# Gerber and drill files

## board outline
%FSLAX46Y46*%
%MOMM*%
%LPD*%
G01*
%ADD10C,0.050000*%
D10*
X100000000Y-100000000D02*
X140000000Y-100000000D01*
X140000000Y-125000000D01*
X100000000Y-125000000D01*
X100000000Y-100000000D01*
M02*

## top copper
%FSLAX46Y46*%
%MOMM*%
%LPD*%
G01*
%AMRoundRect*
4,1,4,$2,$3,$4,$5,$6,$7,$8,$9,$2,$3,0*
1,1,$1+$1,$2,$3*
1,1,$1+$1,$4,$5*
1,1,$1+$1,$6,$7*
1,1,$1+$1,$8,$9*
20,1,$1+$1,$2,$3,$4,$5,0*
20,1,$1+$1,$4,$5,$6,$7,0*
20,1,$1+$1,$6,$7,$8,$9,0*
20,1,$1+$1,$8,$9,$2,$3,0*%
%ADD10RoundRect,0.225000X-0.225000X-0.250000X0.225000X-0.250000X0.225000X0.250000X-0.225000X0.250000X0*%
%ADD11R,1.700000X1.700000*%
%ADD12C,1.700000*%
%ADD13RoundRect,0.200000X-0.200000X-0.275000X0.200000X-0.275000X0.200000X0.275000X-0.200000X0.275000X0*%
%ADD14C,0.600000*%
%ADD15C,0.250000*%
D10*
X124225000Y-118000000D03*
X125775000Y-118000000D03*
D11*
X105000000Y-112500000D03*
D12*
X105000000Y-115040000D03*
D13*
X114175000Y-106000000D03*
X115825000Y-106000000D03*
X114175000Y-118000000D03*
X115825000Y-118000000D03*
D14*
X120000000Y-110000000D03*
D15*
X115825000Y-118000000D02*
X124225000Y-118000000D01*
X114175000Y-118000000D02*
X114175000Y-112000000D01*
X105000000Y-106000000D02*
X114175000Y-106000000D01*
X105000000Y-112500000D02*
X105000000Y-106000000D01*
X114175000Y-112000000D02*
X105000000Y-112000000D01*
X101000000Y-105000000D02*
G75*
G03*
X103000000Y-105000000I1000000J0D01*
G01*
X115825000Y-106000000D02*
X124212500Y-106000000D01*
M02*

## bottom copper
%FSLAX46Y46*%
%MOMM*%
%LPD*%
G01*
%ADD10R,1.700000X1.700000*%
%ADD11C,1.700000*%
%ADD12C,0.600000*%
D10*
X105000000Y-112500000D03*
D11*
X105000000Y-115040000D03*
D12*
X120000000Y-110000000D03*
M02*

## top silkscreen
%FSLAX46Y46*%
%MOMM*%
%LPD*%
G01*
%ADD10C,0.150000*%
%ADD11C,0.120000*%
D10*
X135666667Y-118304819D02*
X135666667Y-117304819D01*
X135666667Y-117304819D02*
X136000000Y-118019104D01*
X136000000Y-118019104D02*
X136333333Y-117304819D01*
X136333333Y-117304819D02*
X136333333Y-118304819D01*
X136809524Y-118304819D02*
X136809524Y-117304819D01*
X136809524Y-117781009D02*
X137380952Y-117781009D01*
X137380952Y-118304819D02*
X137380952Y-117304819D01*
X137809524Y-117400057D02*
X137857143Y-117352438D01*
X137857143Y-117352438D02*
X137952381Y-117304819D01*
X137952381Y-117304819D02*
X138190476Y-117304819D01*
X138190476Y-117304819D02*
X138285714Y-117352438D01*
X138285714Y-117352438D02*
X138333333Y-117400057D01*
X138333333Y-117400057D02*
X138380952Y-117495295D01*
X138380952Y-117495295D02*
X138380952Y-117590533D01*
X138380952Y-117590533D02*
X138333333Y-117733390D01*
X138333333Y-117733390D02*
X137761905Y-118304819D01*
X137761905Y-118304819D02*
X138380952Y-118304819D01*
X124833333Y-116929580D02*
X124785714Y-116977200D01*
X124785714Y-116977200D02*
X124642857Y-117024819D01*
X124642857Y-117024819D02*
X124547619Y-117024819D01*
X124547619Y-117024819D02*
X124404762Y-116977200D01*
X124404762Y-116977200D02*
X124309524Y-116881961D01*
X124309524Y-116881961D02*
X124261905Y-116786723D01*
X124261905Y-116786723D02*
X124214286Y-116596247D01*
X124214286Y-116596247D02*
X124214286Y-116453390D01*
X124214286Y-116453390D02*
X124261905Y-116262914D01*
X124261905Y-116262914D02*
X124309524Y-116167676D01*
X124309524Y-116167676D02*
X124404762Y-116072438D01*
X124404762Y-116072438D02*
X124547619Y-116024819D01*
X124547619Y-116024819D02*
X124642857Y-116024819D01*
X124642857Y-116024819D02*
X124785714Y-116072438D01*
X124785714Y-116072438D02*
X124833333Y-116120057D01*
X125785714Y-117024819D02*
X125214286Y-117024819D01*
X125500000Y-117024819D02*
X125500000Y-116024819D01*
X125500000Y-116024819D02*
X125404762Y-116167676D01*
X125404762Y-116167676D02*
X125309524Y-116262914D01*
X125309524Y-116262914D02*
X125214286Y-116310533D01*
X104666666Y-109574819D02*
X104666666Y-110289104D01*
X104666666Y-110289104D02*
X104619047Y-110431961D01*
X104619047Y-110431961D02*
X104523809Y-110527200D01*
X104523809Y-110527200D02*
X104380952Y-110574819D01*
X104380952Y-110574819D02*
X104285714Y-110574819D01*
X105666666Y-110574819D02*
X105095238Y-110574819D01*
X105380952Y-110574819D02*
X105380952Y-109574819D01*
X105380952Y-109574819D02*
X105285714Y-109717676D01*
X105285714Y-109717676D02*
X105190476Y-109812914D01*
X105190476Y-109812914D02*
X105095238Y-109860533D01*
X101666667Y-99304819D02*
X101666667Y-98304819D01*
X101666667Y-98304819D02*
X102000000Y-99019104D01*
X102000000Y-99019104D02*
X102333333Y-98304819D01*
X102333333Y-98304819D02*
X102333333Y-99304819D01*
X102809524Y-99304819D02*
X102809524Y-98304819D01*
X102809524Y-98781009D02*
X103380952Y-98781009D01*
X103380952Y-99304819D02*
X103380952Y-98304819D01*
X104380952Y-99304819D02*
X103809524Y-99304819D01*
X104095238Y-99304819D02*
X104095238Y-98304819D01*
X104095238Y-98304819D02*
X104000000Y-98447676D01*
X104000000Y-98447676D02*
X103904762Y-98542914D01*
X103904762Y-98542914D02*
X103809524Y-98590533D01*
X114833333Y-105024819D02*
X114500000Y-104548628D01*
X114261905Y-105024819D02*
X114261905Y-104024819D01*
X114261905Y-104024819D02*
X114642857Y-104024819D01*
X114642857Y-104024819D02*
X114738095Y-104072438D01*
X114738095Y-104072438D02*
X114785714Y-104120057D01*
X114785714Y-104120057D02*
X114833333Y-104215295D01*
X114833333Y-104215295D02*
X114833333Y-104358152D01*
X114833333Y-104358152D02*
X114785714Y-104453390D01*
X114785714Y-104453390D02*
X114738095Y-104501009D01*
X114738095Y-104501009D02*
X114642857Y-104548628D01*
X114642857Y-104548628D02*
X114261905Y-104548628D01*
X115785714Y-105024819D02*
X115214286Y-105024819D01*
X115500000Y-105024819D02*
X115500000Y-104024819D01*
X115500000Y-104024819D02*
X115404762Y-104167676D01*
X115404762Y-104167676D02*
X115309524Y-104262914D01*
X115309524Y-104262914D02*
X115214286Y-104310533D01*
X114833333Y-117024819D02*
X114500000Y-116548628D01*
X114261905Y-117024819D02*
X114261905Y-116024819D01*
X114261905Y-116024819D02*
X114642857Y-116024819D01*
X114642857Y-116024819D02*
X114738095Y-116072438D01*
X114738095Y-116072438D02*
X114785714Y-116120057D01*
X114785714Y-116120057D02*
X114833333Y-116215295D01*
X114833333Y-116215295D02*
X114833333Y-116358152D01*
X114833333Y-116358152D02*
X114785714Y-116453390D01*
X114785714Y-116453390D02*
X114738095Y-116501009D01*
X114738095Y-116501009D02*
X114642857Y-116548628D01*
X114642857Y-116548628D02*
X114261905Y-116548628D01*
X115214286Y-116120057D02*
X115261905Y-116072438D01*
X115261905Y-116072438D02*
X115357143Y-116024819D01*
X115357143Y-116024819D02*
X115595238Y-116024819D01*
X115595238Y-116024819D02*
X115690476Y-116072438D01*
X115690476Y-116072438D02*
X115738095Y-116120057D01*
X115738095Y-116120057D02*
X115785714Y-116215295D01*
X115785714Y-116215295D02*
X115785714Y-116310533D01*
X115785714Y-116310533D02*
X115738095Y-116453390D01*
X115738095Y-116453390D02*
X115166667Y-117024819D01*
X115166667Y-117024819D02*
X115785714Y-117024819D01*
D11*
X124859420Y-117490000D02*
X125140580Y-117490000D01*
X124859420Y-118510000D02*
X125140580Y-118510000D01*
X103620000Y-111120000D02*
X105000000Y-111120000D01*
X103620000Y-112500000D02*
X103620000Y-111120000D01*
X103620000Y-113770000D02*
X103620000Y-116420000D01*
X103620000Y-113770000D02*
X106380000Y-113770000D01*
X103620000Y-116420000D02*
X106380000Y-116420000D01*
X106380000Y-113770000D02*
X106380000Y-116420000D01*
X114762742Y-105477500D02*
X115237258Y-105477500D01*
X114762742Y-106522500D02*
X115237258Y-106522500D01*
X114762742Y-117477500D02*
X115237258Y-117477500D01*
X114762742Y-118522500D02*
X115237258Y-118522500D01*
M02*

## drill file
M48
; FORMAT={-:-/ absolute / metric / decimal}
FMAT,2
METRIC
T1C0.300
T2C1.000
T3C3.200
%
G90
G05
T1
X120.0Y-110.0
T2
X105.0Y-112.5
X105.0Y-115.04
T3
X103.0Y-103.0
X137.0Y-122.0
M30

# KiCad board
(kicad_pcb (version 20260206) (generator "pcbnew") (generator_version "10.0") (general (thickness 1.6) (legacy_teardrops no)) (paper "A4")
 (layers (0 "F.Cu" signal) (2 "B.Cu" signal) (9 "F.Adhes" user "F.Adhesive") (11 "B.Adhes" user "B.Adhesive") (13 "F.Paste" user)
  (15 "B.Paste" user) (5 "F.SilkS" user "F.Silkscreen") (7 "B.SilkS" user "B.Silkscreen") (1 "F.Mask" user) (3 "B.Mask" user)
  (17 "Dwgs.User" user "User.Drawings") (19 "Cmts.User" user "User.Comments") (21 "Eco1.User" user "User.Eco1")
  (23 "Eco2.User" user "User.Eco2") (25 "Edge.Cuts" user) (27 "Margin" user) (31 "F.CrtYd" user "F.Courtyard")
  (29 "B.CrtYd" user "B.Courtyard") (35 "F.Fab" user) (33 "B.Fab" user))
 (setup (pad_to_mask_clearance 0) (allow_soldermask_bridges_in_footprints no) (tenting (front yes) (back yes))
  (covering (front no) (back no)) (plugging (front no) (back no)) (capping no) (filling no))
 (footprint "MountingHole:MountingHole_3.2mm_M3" (layer "F.Cu") (at 137 122)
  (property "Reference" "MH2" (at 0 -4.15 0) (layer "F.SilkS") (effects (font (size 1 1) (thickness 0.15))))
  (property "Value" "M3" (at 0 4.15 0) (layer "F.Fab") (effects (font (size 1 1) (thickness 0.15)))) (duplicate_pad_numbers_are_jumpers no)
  (pad "" np_thru_hole circle (at 0 0) (size 3.2 3.2) (drill 3.2) (layers "*.Cu" "*.Mask")))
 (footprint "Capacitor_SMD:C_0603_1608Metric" (layer "F.Cu") (at 125 118)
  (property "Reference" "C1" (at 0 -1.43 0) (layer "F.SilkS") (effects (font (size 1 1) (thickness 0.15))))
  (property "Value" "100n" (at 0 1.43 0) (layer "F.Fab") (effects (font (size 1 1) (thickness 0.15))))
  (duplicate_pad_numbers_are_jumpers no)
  (fp_line (start -0.14058 -0.51) (end 0.14058 -0.51) (stroke (width 0.12) (type solid)) (layer "F.SilkS"))
  (fp_line (start -0.14058 0.51) (end 0.14058 0.51) (stroke (width 0.12) (type solid)) (layer "F.SilkS"))
  (pad "1" smd roundrect (at -0.775 0) (size 0.9 0.95) (layers "F.Cu" "F.Mask" "F.Paste") (roundrect_rratio 0.25) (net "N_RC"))
  (pad "2" smd roundrect (at 0.775 0) (size 0.9 0.95) (layers "F.Cu" "F.Mask" "F.Paste") (roundrect_rratio 0.25) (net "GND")))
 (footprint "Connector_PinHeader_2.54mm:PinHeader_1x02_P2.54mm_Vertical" (layer "F.Cu") (at 105 112.5)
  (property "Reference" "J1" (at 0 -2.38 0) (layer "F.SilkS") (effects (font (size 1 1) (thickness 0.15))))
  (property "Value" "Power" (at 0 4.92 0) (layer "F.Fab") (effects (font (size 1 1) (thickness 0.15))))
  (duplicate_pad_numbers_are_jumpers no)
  (fp_line (start -1.38 -1.38) (end 0 -1.38) (stroke (width 0.12) (type solid)) (layer "F.SilkS"))
  (fp_line (start -1.38 0) (end -1.38 -1.38) (stroke (width 0.12) (type solid)) (layer "F.SilkS"))
  (fp_line (start -1.38 1.27) (end -1.38 3.92) (stroke (width 0.12) (type solid)) (layer "F.SilkS"))
  (fp_line (start -1.38 1.27) (end 1.38 1.27) (stroke (width 0.12) (type solid)) (layer "F.SilkS"))
  (fp_line (start -1.38 3.92) (end 1.38 3.92) (stroke (width 0.12) (type solid)) (layer "F.SilkS"))
  (fp_line (start 1.38 1.27) (end 1.38 3.92) (stroke (width 0.12) (type solid)) (layer "F.SilkS"))
  (pad "1" thru_hole rect (at 0 0) (size 1.7 1.7) (drill 1) (layers "*.Cu" "*.Mask") (remove_unused_layers no) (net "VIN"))
  (pad "2" thru_hole circle (at 0 2.54) (size 1.7 1.7) (drill 1) (layers "*.Cu" "*.Mask") (remove_unused_layers no) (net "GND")))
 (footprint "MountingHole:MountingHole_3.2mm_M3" (layer "F.Cu") (at 103 103)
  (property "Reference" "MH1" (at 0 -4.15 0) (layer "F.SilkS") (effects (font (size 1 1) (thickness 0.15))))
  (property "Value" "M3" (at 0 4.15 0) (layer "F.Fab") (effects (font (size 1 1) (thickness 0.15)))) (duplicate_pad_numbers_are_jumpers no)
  (pad "" np_thru_hole circle (at 0 0) (size 3.2 3.2) (drill 3.2) (layers "*.Cu" "*.Mask")))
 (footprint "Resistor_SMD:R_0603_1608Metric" (layer "F.Cu") (at 115 106)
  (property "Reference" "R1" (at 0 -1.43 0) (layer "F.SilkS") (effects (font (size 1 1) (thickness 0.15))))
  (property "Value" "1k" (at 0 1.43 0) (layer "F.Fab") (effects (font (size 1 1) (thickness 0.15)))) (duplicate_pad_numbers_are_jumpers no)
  (fp_line (start -0.237258 -0.5225) (end 0.237258 -0.5225) (stroke (width 0.12) (type solid)) (layer "F.SilkS"))
  (fp_line (start -0.237258 0.5225) (end 0.237258 0.5225) (stroke (width 0.12) (type solid)) (layer "F.SilkS"))
  (pad "1" smd roundrect (at -0.825 0) (size 0.8 0.95) (layers "F.Cu" "F.Mask" "F.Paste") (roundrect_rratio 0.25) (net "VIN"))
  (pad "2" smd roundrect (at 0.825 0) (size 0.8 0.95) (layers "F.Cu" "F.Mask" "F.Paste") (roundrect_rratio 0.25) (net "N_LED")))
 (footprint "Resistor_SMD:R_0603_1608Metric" (layer "F.Cu") (at 115 118)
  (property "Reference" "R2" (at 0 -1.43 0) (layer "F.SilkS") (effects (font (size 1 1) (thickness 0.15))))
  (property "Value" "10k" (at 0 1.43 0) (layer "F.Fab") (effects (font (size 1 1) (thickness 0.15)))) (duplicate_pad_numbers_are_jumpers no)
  (fp_line (start -0.237258 -0.5225) (end 0.237258 -0.5225) (stroke (width 0.12) (type solid)) (layer "F.SilkS"))
  (fp_line (start -0.237258 0.5225) (end 0.237258 0.5225) (stroke (width 0.12) (type solid)) (layer "F.SilkS"))
  (pad "1" smd roundrect (at -0.825 0) (size 0.8 0.95) (layers "F.Cu" "F.Mask" "F.Paste") (roundrect_rratio 0.25) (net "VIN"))
  (pad "2" smd roundrect (at 0.825 0) (size 0.8 0.95) (layers "F.Cu" "F.Mask" "F.Paste") (roundrect_rratio 0.25) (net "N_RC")))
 (gr_rect (start 100 100) (end 140 125) (stroke (width 0.05) (type default)) (fill no) (layer "Edge.Cuts"))
 (segment (start 115.825 118) (end 124.225 118) (width 0.25) (layer "F.Cu") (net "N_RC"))
 (segment (start 114.175 118) (end 114.175 112) (width 0.25) (layer "F.Cu") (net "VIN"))
 (segment (start 105 106) (end 114.175 106) (width 0.25) (layer "F.Cu") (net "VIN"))
 (segment (start 105 112.5) (end 105 106) (width 0.25) (layer "F.Cu") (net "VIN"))
 (segment (start 114.175 112) (end 105 112) (width 0.25) (layer "F.Cu") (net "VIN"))
 (via (at 120 110) (size 0.6) (drill 0.3) (layers "F.Cu" "B.Cu") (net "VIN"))
 (arc (start 101 105) (mid 102 106) (end 103 105) (width 0.25) (layer "F.Cu") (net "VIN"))
 (segment (start 115.825 106) (end 124.2125 106) (width 0.25) (layer "F.Cu") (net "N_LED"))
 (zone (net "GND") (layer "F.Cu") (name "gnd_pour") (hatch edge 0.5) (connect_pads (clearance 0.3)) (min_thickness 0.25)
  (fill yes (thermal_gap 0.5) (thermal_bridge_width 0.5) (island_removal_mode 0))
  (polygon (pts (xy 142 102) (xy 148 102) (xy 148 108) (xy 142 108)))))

